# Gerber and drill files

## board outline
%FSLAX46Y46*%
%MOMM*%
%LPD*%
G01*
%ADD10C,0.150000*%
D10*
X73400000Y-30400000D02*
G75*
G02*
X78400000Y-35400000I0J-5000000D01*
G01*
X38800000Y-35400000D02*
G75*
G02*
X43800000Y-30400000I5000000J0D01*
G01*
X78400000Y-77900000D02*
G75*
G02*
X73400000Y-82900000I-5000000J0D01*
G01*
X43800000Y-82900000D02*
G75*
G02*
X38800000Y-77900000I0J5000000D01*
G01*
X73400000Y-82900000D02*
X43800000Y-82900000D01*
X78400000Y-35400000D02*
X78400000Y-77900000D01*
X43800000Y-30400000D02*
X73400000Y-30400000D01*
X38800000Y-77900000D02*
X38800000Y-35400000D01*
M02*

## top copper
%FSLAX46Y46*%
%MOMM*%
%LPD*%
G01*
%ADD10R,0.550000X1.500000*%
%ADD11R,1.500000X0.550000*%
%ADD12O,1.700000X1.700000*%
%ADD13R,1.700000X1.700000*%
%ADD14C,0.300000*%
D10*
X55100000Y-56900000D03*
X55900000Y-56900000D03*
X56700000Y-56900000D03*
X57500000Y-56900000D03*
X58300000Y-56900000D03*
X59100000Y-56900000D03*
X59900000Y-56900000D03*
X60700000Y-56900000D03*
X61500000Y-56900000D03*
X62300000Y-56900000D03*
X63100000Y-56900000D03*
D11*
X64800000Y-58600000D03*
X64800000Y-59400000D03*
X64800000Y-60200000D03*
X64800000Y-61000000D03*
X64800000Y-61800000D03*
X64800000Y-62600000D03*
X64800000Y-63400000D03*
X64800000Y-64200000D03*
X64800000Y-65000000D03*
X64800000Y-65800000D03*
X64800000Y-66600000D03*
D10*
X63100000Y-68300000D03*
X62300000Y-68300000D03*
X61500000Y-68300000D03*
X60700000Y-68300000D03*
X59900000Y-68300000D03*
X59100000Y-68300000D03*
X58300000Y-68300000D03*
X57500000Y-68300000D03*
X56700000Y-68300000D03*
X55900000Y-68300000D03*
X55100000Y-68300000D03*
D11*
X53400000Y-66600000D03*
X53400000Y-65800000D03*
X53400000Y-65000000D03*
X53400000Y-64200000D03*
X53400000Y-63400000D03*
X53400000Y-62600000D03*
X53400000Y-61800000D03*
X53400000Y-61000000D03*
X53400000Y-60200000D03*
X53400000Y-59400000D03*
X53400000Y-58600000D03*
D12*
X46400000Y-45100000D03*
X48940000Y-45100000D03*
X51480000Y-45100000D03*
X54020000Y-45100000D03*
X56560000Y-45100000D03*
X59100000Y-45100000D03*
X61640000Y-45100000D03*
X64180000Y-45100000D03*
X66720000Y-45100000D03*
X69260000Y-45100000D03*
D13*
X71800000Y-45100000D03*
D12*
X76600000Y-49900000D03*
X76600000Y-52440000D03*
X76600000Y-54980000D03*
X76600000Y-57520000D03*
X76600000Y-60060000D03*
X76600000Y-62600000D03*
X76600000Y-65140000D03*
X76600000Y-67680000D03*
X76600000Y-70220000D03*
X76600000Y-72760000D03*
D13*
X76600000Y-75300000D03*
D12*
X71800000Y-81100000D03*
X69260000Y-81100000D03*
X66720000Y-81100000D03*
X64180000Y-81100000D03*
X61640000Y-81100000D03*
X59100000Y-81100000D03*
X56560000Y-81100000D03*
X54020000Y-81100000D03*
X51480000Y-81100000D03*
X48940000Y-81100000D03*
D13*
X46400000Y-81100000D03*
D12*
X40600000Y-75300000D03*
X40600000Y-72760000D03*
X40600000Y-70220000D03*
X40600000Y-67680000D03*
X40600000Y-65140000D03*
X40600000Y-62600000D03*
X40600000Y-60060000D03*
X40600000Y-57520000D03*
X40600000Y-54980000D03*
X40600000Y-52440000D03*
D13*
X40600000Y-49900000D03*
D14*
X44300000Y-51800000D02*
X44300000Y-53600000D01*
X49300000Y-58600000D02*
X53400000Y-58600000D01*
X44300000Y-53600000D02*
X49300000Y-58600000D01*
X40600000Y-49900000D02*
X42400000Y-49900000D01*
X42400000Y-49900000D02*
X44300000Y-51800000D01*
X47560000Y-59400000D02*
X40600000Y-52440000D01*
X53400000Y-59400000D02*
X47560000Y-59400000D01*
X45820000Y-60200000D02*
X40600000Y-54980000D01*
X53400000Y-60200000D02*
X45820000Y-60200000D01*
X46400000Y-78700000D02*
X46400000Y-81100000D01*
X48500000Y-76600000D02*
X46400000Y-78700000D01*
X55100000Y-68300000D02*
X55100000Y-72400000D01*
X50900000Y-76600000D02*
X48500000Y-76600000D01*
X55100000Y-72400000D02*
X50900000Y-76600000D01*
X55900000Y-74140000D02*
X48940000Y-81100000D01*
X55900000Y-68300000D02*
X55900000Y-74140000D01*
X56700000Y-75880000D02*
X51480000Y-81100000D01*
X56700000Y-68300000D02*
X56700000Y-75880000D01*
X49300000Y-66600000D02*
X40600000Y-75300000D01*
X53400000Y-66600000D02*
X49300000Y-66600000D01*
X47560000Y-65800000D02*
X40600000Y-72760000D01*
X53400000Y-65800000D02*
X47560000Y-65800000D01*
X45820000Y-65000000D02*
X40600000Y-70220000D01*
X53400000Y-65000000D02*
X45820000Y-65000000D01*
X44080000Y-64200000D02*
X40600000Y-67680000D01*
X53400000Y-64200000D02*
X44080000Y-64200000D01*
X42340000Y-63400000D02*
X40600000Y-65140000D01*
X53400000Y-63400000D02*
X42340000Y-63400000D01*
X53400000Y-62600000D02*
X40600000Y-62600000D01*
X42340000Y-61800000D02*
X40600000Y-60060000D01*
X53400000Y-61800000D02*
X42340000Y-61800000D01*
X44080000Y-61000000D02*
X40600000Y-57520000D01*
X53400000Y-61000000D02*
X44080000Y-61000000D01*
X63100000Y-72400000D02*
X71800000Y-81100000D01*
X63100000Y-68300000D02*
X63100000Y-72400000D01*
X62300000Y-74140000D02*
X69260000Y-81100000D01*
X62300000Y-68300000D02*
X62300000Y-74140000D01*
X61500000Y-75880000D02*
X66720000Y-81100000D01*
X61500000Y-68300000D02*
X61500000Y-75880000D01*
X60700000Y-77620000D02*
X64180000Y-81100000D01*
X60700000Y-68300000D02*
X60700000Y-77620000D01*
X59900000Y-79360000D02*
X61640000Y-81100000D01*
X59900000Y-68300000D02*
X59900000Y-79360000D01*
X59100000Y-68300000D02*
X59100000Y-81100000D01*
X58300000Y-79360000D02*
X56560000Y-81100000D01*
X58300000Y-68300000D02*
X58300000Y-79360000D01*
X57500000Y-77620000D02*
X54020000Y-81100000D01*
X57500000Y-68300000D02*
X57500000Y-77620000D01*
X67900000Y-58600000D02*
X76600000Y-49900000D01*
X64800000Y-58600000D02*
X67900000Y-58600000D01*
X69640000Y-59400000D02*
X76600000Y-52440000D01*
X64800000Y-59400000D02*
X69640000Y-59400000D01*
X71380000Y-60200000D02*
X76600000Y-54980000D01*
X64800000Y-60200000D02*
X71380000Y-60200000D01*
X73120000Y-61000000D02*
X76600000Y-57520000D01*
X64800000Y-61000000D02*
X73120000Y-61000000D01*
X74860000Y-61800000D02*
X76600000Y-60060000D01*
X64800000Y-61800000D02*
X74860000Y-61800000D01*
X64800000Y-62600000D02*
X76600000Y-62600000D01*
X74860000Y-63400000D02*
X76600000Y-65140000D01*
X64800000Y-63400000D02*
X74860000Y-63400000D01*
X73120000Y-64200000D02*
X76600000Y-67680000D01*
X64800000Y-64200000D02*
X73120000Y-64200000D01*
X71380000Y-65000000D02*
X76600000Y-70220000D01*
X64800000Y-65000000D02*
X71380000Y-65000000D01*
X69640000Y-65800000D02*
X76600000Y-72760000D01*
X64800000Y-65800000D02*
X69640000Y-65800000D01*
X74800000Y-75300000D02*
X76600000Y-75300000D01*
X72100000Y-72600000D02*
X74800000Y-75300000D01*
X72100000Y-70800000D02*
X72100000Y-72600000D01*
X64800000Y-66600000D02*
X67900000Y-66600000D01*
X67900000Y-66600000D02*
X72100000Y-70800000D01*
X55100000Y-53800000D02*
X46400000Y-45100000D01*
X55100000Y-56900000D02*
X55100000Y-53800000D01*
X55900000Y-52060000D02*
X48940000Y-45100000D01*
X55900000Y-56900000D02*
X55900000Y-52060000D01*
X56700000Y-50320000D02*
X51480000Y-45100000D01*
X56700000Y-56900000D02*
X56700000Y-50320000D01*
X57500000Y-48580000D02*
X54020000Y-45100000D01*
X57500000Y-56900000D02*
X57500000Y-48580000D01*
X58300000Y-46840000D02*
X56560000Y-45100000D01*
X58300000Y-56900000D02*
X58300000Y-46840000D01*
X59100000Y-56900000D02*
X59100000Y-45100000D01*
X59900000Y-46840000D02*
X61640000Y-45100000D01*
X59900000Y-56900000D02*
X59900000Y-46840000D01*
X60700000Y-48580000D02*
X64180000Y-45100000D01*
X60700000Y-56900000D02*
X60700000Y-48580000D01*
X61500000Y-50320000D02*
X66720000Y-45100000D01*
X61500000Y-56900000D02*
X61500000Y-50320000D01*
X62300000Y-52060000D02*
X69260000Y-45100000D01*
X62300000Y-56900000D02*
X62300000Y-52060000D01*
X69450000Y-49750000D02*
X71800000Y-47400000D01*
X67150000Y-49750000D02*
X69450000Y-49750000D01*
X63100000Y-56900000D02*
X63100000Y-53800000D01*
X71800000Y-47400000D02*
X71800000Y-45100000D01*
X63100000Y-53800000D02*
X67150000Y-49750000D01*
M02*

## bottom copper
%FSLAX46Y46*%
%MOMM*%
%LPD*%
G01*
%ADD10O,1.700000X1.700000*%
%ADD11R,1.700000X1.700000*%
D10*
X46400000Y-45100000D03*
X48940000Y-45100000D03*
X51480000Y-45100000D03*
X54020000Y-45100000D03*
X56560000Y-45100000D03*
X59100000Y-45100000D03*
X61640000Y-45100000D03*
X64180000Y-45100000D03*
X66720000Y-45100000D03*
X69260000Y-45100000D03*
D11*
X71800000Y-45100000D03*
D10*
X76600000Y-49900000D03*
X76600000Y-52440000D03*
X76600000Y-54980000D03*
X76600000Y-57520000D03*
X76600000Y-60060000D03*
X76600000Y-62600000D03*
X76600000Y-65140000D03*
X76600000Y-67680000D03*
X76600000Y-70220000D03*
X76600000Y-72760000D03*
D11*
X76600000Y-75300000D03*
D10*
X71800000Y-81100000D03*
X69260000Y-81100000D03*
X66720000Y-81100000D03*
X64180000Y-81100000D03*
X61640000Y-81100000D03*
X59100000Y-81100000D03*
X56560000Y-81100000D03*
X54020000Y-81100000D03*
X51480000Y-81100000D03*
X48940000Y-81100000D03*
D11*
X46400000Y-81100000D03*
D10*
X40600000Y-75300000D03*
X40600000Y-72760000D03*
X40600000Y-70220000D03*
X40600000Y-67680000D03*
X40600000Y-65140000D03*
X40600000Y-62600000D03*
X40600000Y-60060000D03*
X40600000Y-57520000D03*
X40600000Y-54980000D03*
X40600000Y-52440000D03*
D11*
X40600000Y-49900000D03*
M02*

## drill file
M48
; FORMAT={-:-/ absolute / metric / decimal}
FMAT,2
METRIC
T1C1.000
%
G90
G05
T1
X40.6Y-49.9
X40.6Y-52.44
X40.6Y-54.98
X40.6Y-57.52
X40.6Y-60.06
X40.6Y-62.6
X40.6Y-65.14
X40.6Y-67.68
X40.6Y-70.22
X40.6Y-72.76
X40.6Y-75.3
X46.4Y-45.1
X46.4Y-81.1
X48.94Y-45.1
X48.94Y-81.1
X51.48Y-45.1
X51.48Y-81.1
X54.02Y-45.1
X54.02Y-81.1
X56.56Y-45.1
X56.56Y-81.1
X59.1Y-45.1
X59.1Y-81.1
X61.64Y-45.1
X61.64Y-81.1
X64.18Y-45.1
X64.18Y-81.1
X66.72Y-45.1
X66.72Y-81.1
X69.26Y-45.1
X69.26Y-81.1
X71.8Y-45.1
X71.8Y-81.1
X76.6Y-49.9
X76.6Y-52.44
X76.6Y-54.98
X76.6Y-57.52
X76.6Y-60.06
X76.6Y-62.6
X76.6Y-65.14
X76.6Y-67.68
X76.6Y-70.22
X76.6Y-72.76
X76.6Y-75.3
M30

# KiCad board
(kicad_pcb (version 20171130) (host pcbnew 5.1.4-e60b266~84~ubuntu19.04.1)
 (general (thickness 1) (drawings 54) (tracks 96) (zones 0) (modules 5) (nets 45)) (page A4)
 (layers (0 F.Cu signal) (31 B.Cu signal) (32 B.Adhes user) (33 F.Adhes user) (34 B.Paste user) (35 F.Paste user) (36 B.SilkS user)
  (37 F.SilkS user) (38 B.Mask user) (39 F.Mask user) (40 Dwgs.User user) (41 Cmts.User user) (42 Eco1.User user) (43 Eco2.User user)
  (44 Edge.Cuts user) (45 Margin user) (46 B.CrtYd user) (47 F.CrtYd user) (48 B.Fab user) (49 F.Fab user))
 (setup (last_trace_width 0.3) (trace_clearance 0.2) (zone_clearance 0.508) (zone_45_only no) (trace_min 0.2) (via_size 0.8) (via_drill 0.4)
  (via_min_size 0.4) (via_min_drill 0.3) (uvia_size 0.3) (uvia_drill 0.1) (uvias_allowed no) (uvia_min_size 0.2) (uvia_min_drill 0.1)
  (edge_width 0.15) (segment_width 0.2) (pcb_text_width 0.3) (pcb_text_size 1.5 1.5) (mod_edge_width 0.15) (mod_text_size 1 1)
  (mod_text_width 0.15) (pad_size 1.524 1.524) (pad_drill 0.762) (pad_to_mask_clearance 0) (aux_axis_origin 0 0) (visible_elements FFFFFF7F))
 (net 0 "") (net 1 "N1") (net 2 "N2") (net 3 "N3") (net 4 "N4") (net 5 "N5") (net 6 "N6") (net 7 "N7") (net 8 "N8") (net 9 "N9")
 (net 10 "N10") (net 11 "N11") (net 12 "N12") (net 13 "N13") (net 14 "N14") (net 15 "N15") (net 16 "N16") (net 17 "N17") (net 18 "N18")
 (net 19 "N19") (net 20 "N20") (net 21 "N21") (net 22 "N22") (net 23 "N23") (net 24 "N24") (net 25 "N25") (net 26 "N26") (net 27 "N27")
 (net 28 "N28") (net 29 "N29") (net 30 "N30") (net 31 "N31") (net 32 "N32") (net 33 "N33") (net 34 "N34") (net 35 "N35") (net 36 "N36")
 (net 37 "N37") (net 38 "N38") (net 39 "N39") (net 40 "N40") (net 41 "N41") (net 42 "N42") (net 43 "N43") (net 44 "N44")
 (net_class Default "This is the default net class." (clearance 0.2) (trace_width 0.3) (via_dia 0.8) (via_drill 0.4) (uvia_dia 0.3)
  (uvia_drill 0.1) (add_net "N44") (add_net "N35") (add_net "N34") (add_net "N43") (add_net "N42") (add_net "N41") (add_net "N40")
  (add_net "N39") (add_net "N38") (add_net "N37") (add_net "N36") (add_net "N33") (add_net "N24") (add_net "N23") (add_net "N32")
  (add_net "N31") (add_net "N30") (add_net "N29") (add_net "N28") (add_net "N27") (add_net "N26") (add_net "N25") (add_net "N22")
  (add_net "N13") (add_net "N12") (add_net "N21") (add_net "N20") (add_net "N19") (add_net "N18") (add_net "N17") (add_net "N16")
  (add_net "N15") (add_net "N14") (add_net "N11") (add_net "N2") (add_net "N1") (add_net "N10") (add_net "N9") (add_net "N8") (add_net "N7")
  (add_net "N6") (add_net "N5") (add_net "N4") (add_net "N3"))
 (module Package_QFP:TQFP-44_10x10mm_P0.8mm (layer F.Cu) (at 59.1 62.6)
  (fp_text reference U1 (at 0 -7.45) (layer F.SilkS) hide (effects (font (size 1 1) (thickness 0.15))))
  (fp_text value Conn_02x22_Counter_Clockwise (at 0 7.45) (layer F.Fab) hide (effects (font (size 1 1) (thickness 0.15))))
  (pad 44 smd rect (at -4 -5.7 90) (size 1.5 0.55) (layers F.Cu F.Paste F.Mask) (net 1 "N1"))
  (pad 43 smd rect (at -3.2 -5.7 90) (size 1.5 0.55) (layers F.Cu F.Paste F.Mask) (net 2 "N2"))
  (pad 42 smd rect (at -2.4 -5.7 90) (size 1.5 0.55) (layers F.Cu F.Paste F.Mask) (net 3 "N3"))
  (pad 41 smd rect (at -1.6 -5.7 90) (size 1.5 0.55) (layers F.Cu F.Paste F.Mask) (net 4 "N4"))
  (pad 40 smd rect (at -0.8 -5.7 90) (size 1.5 0.55) (layers F.Cu F.Paste F.Mask) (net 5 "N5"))
  (pad 39 smd rect (at 0 -5.7 90) (size 1.5 0.55) (layers F.Cu F.Paste F.Mask) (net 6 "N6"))
  (pad 38 smd rect (at 0.8 -5.7 90) (size 1.5 0.55) (layers F.Cu F.Paste F.Mask) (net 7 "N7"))
  (pad 37 smd rect (at 1.6 -5.7 90) (size 1.5 0.55) (layers F.Cu F.Paste F.Mask) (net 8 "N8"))
  (pad 36 smd rect (at 2.4 -5.7 90) (size 1.5 0.55) (layers F.Cu F.Paste F.Mask) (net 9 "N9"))
  (pad 35 smd rect (at 3.2 -5.7 90) (size 1.5 0.55) (layers F.Cu F.Paste F.Mask) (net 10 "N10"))
  (pad 34 smd rect (at 4 -5.7 90) (size 1.5 0.55) (layers F.Cu F.Paste F.Mask) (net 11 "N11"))
  (pad 33 smd rect (at 5.7 -4) (size 1.5 0.55) (layers F.Cu F.Paste F.Mask) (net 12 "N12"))
  (pad 32 smd rect (at 5.7 -3.2) (size 1.5 0.55) (layers F.Cu F.Paste F.Mask) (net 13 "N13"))
  (pad 31 smd rect (at 5.7 -2.4) (size 1.5 0.55) (layers F.Cu F.Paste F.Mask) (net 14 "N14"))
  (pad 30 smd rect (at 5.7 -1.6) (size 1.5 0.55) (layers F.Cu F.Paste F.Mask) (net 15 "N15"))
  (pad 29 smd rect (at 5.7 -0.8) (size 1.5 0.55) (layers F.Cu F.Paste F.Mask) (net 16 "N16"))
  (pad 28 smd rect (at 5.7 0) (size 1.5 0.55) (layers F.Cu F.Paste F.Mask) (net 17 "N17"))
  (pad 27 smd rect (at 5.7 0.8) (size 1.5 0.55) (layers F.Cu F.Paste F.Mask) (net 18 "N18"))
  (pad 26 smd rect (at 5.7 1.6) (size 1.5 0.55) (layers F.Cu F.Paste F.Mask) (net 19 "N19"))
  (pad 25 smd rect (at 5.7 2.4) (size 1.5 0.55) (layers F.Cu F.Paste F.Mask) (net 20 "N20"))
  (pad 24 smd rect (at 5.7 3.2) (size 1.5 0.55) (layers F.Cu F.Paste F.Mask) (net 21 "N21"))
  (pad 23 smd rect (at 5.7 4) (size 1.5 0.55) (layers F.Cu F.Paste F.Mask) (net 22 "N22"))
  (pad 22 smd rect (at 4 5.7 90) (size 1.5 0.55) (layers F.Cu F.Paste F.Mask) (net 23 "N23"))
  (pad 21 smd rect (at 3.2 5.7 90) (size 1.5 0.55) (layers F.Cu F.Paste F.Mask) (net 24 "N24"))
  (pad 20 smd rect (at 2.4 5.7 90) (size 1.5 0.55) (layers F.Cu F.Paste F.Mask) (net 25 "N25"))
  (pad 19 smd rect (at 1.6 5.7 90) (size 1.5 0.55) (layers F.Cu F.Paste F.Mask) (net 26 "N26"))
  (pad 18 smd rect (at 0.8 5.7 90) (size 1.5 0.55) (layers F.Cu F.Paste F.Mask) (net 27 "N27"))
  (pad 17 smd rect (at 0 5.7 90) (size 1.5 0.55) (layers F.Cu F.Paste F.Mask) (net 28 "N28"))
  (pad 16 smd rect (at -0.8 5.7 90) (size 1.5 0.55) (layers F.Cu F.Paste F.Mask) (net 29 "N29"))
  (pad 15 smd rect (at -1.6 5.7 90) (size 1.5 0.55) (layers F.Cu F.Paste F.Mask) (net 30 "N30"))
  (pad 14 smd rect (at -2.4 5.7 90) (size 1.5 0.55) (layers F.Cu F.Paste F.Mask) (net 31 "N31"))
  (pad 13 smd rect (at -3.2 5.7 90) (size 1.5 0.55) (layers F.Cu F.Paste F.Mask) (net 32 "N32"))
  (pad 12 smd rect (at -4 5.7 90) (size 1.5 0.55) (layers F.Cu F.Paste F.Mask) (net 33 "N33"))
  (pad 11 smd rect (at -5.7 4) (size 1.5 0.55) (layers F.Cu F.Paste F.Mask) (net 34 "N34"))
  (pad 10 smd rect (at -5.7 3.2) (size 1.5 0.55) (layers F.Cu F.Paste F.Mask) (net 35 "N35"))
  (pad 9 smd rect (at -5.7 2.4) (size 1.5 0.55) (layers F.Cu F.Paste F.Mask) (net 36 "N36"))
  (pad 8 smd rect (at -5.7 1.6) (size 1.5 0.55) (layers F.Cu F.Paste F.Mask) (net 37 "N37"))
  (pad 7 smd rect (at -5.7 0.8) (size 1.5 0.55) (layers F.Cu F.Paste F.Mask) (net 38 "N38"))
  (pad 6 smd rect (at -5.7 0) (size 1.5 0.55) (layers F.Cu F.Paste F.Mask) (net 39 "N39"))
  (pad 5 smd rect (at -5.7 -0.8) (size 1.5 0.55) (layers F.Cu F.Paste F.Mask) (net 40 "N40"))
  (pad 4 smd rect (at -5.7 -1.6) (size 1.5 0.55) (layers F.Cu F.Paste F.Mask) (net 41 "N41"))
  (pad 3 smd rect (at -5.7 -2.4) (size 1.5 0.55) (layers F.Cu F.Paste F.Mask) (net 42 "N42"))
  (pad 2 smd rect (at -5.7 -3.2) (size 1.5 0.55) (layers F.Cu F.Paste F.Mask) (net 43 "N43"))
  (pad 1 smd rect (at -5.7 -4) (size 1.5 0.55) (layers F.Cu F.Paste F.Mask) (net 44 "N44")))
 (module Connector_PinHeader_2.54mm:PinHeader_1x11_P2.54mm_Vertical (layer F.Cu) (at 71.8 45.1 270)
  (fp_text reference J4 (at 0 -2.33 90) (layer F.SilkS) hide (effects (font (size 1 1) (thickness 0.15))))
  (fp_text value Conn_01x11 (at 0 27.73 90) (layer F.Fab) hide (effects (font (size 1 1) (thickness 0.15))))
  (pad 11 thru_hole oval (at 0 25.4 270) (size 1.7 1.7) (drill 1) (layers *.Cu *.Mask) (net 1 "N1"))
  (pad 10 thru_hole oval (at 0 22.86 270) (size 1.7 1.7) (drill 1) (layers *.Cu *.Mask) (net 2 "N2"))
  (pad 9 thru_hole oval (at 0 20.32 270) (size 1.7 1.7) (drill 1) (layers *.Cu *.Mask) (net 3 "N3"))
  (pad 8 thru_hole oval (at 0 17.78 270) (size 1.7 1.7) (drill 1) (layers *.Cu *.Mask) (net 4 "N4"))
  (pad 7 thru_hole oval (at 0 15.24 270) (size 1.7 1.7) (drill 1) (layers *.Cu *.Mask) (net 5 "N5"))
  (pad 6 thru_hole oval (at 0 12.7 270) (size 1.7 1.7) (drill 1) (layers *.Cu *.Mask) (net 6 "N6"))
  (pad 5 thru_hole oval (at 0 10.16 270) (size 1.7 1.7) (drill 1) (layers *.Cu *.Mask) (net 7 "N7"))
  (pad 4 thru_hole oval (at 0 7.62 270) (size 1.7 1.7) (drill 1) (layers *.Cu *.Mask) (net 8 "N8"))
  (pad 3 thru_hole oval (at 0 5.08 270) (size 1.7 1.7) (drill 1) (layers *.Cu *.Mask) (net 9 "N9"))
  (pad 2 thru_hole oval (at 0 2.54 270) (size 1.7 1.7) (drill 1) (layers *.Cu *.Mask) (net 10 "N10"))
  (pad 1 thru_hole rect (at 0 0 270) (size 1.7 1.7) (drill 1) (layers *.Cu *.Mask) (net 11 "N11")))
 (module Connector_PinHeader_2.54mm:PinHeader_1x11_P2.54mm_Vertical (layer F.Cu) (at 76.6 75.3 180)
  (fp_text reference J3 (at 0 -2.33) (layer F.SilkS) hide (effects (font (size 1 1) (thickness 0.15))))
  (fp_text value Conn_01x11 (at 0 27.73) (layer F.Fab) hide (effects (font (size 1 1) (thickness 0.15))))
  (pad 11 thru_hole oval (at 0 25.4 180) (size 1.7 1.7) (drill 1) (layers *.Cu *.Mask) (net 12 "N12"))
  (pad 10 thru_hole oval (at 0 22.86 180) (size 1.7 1.7) (drill 1) (layers *.Cu *.Mask) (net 13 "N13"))
  (pad 9 thru_hole oval (at 0 20.32 180) (size 1.7 1.7) (drill 1) (layers *.Cu *.Mask) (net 14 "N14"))
  (pad 8 thru_hole oval (at 0 17.78 180) (size 1.7 1.7) (drill 1) (layers *.Cu *.Mask) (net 15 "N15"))
  (pad 7 thru_hole oval (at 0 15.24 180) (size 1.7 1.7) (drill 1) (layers *.Cu *.Mask) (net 16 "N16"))
  (pad 6 thru_hole oval (at 0 12.7 180) (size 1.7 1.7) (drill 1) (layers *.Cu *.Mask) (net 17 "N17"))
  (pad 5 thru_hole oval (at 0 10.16 180) (size 1.7 1.7) (drill 1) (layers *.Cu *.Mask) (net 18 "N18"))
  (pad 4 thru_hole oval (at 0 7.62 180) (size 1.7 1.7) (drill 1) (layers *.Cu *.Mask) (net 19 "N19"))
  (pad 3 thru_hole oval (at 0 5.08 180) (size 1.7 1.7) (drill 1) (layers *.Cu *.Mask) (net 20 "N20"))
  (pad 2 thru_hole oval (at 0 2.54 180) (size 1.7 1.7) (drill 1) (layers *.Cu *.Mask) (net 21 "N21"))
  (pad 1 thru_hole rect (at 0 0 180) (size 1.7 1.7) (drill 1) (layers *.Cu *.Mask) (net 22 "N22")))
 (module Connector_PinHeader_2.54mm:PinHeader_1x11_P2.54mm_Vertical (layer F.Cu) (at 46.4 81.1 90)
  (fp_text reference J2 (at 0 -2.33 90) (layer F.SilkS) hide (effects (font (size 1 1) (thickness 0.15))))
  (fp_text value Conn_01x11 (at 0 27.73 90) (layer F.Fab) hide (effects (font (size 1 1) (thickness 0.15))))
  (pad 11 thru_hole oval (at 0 25.4 90) (size 1.7 1.7) (drill 1) (layers *.Cu *.Mask) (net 23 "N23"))
  (pad 10 thru_hole oval (at 0 22.86 90) (size 1.7 1.7) (drill 1) (layers *.Cu *.Mask) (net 24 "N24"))
  (pad 9 thru_hole oval (at 0 20.32 90) (size 1.7 1.7) (drill 1) (layers *.Cu *.Mask) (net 25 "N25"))
  (pad 8 thru_hole oval (at 0 17.78 90) (size 1.7 1.7) (drill 1) (layers *.Cu *.Mask) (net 26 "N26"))
  (pad 7 thru_hole oval (at 0 15.24 90) (size 1.7 1.7) (drill 1) (layers *.Cu *.Mask) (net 27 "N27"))
  (pad 6 thru_hole oval (at 0 12.7 90) (size 1.7 1.7) (drill 1) (layers *.Cu *.Mask) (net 28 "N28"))
  (pad 5 thru_hole oval (at 0 10.16 90) (size 1.7 1.7) (drill 1) (layers *.Cu *.Mask) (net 29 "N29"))
  (pad 4 thru_hole oval (at 0 7.62 90) (size 1.7 1.7) (drill 1) (layers *.Cu *.Mask) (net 30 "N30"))
  (pad 3 thru_hole oval (at 0 5.08 90) (size 1.7 1.7) (drill 1) (layers *.Cu *.Mask) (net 31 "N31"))
  (pad 2 thru_hole oval (at 0 2.54 90) (size 1.7 1.7) (drill 1) (layers *.Cu *.Mask) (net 32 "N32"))
  (pad 1 thru_hole rect (at 0 0 90) (size 1.7 1.7) (drill 1) (layers *.Cu *.Mask) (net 33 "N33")))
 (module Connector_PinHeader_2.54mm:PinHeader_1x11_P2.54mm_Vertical (layer F.Cu) (at 40.6 49.9)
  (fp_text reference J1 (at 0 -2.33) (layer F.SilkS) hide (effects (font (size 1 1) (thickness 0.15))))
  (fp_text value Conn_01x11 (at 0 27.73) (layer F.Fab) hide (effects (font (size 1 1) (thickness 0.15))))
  (pad 11 thru_hole oval (at 0 25.4) (size 1.7 1.7) (drill 1) (layers *.Cu *.Mask) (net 34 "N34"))
  (pad 10 thru_hole oval (at 0 22.86) (size 1.7 1.7) (drill 1) (layers *.Cu *.Mask) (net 35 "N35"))
  (pad 9 thru_hole oval (at 0 20.32) (size 1.7 1.7) (drill 1) (layers *.Cu *.Mask) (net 36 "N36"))
  (pad 8 thru_hole oval (at 0 17.78) (size 1.7 1.7) (drill 1) (layers *.Cu *.Mask) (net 37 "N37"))
  (pad 7 thru_hole oval (at 0 15.24) (size 1.7 1.7) (drill 1) (layers *.Cu *.Mask) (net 38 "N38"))
  (pad 6 thru_hole oval (at 0 12.7) (size 1.7 1.7) (drill 1) (layers *.Cu *.Mask) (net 39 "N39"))
  (pad 5 thru_hole oval (at 0 10.16) (size 1.7 1.7) (drill 1) (layers *.Cu *.Mask) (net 40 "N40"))
  (pad 4 thru_hole oval (at 0 7.62) (size 1.7 1.7) (drill 1) (layers *.Cu *.Mask) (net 41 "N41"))
  (pad 3 thru_hole oval (at 0 5.08) (size 1.7 1.7) (drill 1) (layers *.Cu *.Mask) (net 42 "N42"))
  (pad 2 thru_hole oval (at 0 2.54) (size 1.7 1.7) (drill 1) (layers *.Cu *.Mask) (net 43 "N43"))
  (pad 1 thru_hole rect (at 0 0) (size 1.7 1.7) (drill 1) (layers *.Cu *.Mask) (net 44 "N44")))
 (gr_arc (start 73.4 35.4) (end 78.4 35.4) (angle -90) (layer Edge.Cuts) (width 0.15))
 (gr_arc (start 43.8 35.4) (end 43.8 30.4) (angle -90) (layer Edge.Cuts) (width 0.15))
 (gr_arc (start 73.4 77.9) (end 73.4 82.9) (angle -90) (layer Edge.Cuts) (width 0.15))
 (gr_arc (start 43.8 77.9) (end 38.8 77.9) (angle -90) (layer Edge.Cuts) (width 0.15))
 (gr_line (start 73.4 82.9) (end 43.8 82.9) (layer Edge.Cuts) (width 0.15))
 (gr_line (start 78.4 35.4) (end 78.4 77.9) (layer Edge.Cuts) (width 0.15))
 (gr_line (start 43.8 30.4) (end 73.4 30.4) (layer Edge.Cuts) (width 0.15))
 (gr_line (start 38.8 77.9) (end 38.8 35.4) (layer Edge.Cuts) (width 0.15))
 (segment (start 44.3 51.8) (end 44.3 53.6) (width 0.3) (layer F.Cu) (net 44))
 (segment (start 49.3 58.6) (end 53.4 58.6) (width 0.3) (layer F.Cu) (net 44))
 (segment (start 44.3 53.6) (end 49.3 58.6) (width 0.3) (layer F.Cu) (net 44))
 (segment (start 40.6 49.9) (end 42.4 49.9) (width 0.3) (layer F.Cu) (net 44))
 (segment (start 42.4 49.9) (end 44.3 51.8) (width 0.3) (layer F.Cu) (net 44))
 (segment (start 47.56 59.4) (end 40.6 52.44) (width 0.3) (layer F.Cu) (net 43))
 (segment (start 53.4 59.4) (end 47.56 59.4) (width 0.3) (layer F.Cu) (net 43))
 (segment (start 45.82 60.2) (end 40.6 54.98) (width 0.3) (layer F.Cu) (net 42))
 (segment (start 53.4 60.2) (end 45.82 60.2) (width 0.3) (layer F.Cu) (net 42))
 (segment (start 46.4 78.7) (end 46.4 81.1) (width 0.3) (layer F.Cu) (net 33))
 (segment (start 48.5 76.6) (end 46.4 78.7) (width 0.3) (layer F.Cu) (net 33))
 (segment (start 55.1 68.3) (end 55.1 72.4) (width 0.3) (layer F.Cu) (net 33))
 (segment (start 50.9 76.6) (end 48.5 76.6) (width 0.3) (layer F.Cu) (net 33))
 (segment (start 55.1 72.4) (end 50.9 76.6) (width 0.3) (layer F.Cu) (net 33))
 (segment (start 55.9 74.14) (end 48.94 81.1) (width 0.3) (layer F.Cu) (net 32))
 (segment (start 55.9 68.3) (end 55.9 74.14) (width 0.3) (layer F.Cu) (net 32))
 (segment (start 56.7 75.88) (end 51.48 81.1) (width 0.3) (layer F.Cu) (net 31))
 (segment (start 56.7 68.3) (end 56.7 75.88) (width 0.3) (layer F.Cu) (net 31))
 (segment (start 49.3 66.6) (end 40.6 75.3) (width 0.3) (layer F.Cu) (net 34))
 (segment (start 53.4 66.6) (end 49.3 66.6) (width 0.3) (layer F.Cu) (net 34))
 (segment (start 47.56 65.8) (end 40.6 72.76) (width 0.3) (layer F.Cu) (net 35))
 (segment (start 53.4 65.8) (end 47.56 65.8) (width 0.3) (layer F.Cu) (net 35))
 (segment (start 45.82 65) (end 40.6 70.22) (width 0.3) (layer F.Cu) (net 36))
 (segment (start 53.4 65) (end 45.82 65) (width 0.3) (layer F.Cu) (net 36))
 (segment (start 44.08 64.2) (end 40.6 67.68) (width 0.3) (layer F.Cu) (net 37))
 (segment (start 53.4 64.2) (end 44.08 64.2) (width 0.3) (layer F.Cu) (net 37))
 (segment (start 42.34 63.4) (end 40.6 65.14) (width 0.3) (layer F.Cu) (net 38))
 (segment (start 53.4 63.4) (end 42.34 63.4) (width 0.3) (layer F.Cu) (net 38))
 (segment (start 53.4 62.6) (end 40.6 62.6) (width 0.3) (layer F.Cu) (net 39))
 (segment (start 42.34 61.8) (end 40.6 60.06) (width 0.3) (layer F.Cu) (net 40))
 (segment (start 53.4 61.8) (end 42.34 61.8) (width 0.3) (layer F.Cu) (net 40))
 (segment (start 44.08 61) (end 40.6 57.52) (width 0.3) (layer F.Cu) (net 41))
 (segment (start 53.4 61) (end 44.08 61) (width 0.3) (layer F.Cu) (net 41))
 (segment (start 63.1 72.4) (end 71.8 81.1) (width 0.3) (layer F.Cu) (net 23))
 (segment (start 63.1 68.3) (end 63.1 72.4) (width 0.3) (layer F.Cu) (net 23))
 (segment (start 62.3 74.14) (end 69.26 81.1) (width 0.3) (layer F.Cu) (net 24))
 (segment (start 62.3 68.3) (end 62.3 74.14) (width 0.3) (layer F.Cu) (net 24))
 (segment (start 61.5 75.88) (end 66.72 81.1) (width 0.3) (layer F.Cu) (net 25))
 (segment (start 61.5 68.3) (end 61.5 75.88) (width 0.3) (layer F.Cu) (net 25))
 (segment (start 60.7 77.62) (end 64.18 81.1) (width 0.3) (layer F.Cu) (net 26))
 (segment (start 60.7 68.3) (end 60.7 77.62) (width 0.3) (layer F.Cu) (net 26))
 (segment (start 59.9 79.36) (end 61.64 81.1) (width 0.3) (layer F.Cu) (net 27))
 (segment (start 59.9 68.3) (end 59.9 79.36) (width 0.3) (layer F.Cu) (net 27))
 (segment (start 59.1 68.3) (end 59.1 81.1) (width 0.3) (layer F.Cu) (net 28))
 (segment (start 58.3 79.36) (end 56.56 81.1) (width 0.3) (layer F.Cu) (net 29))
 (segment (start 58.3 68.3) (end 58.3 79.36) (width 0.3) (layer F.Cu) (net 29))
 (segment (start 57.5 77.62) (end 54.02 81.1) (width 0.3) (layer F.Cu) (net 30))
 (segment (start 57.5 68.3) (end 57.5 77.62) (width 0.3) (layer F.Cu) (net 30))
 (segment (start 67.9 58.6) (end 76.6 49.9) (width 0.3) (layer F.Cu) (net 12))
 (segment (start 64.8 58.6) (end 67.9 58.6) (width 0.3) (layer F.Cu) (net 12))
 (segment (start 69.64 59.4) (end 76.6 52.44) (width 0.3) (layer F.Cu) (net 13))
 (segment (start 64.8 59.4) (end 69.64 59.4) (width 0.3) (layer F.Cu) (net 13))
 (segment (start 71.38 60.2) (end 76.6 54.98) (width 0.3) (layer F.Cu) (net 14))
 (segment (start 64.8 60.2) (end 71.38 60.2) (width 0.3) (layer F.Cu) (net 14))
 (segment (start 73.12 61) (end 76.6 57.52) (width 0.3) (layer F.Cu) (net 15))
 (segment (start 64.8 61) (end 73.12 61) (width 0.3) (layer F.Cu) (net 15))
 (segment (start 74.86 61.8) (end 76.6 60.06) (width 0.3) (layer F.Cu) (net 16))
 (segment (start 64.8 61.8) (end 74.86 61.8) (width 0.3) (layer F.Cu) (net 16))
 (segment (start 64.8 62.6) (end 76.6 62.6) (width 0.3) (layer F.Cu) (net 17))
 (segment (start 74.86 63.4) (end 76.6 65.14) (width 0.3) (layer F.Cu) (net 18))
 (segment (start 64.8 63.4) (end 74.86 63.4) (width 0.3) (layer F.Cu) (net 18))
 (segment (start 73.12 64.2) (end 76.6 67.68) (width 0.3) (layer F.Cu) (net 19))
 (segment (start 64.8 64.2) (end 73.12 64.2) (width 0.3) (layer F.Cu) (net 19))
 (segment (start 71.38 65) (end 76.6 70.22) (width 0.3) (layer F.Cu) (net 20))
 (segment (start 64.8 65) (end 71.38 65) (width 0.3) (layer F.Cu) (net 20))
 (segment (start 69.64 65.8) (end 76.6 72.76) (width 0.3) (layer F.Cu) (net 21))
 (segment (start 64.8 65.8) (end 69.64 65.8) (width 0.3) (layer F.Cu) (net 21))
 (segment (start 74.8 75.3) (end 76.6 75.3) (width 0.3) (layer F.Cu) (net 22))
 (segment (start 72.1 72.6) (end 74.8 75.3) (width 0.3) (layer F.Cu) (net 22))
 (segment (start 72.1 70.8) (end 72.1 72.6) (width 0.3) (layer F.Cu) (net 22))
 (segment (start 64.8 66.6) (end 67.9 66.6) (width 0.3) (layer F.Cu) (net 22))
 (segment (start 67.9 66.6) (end 72.1 70.8) (width 0.3) (layer F.Cu) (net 22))
 (segment (start 55.1 53.8) (end 46.4 45.1) (width 0.3) (layer F.Cu) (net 1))
 (segment (start 55.1 56.9) (end 55.1 53.8) (width 0.3) (layer F.Cu) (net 1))
 (segment (start 55.9 52.06) (end 48.94 45.1) (width 0.3) (layer F.Cu) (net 2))
 (segment (start 55.9 56.9) (end 55.9 52.06) (width 0.3) (layer F.Cu) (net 2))
 (segment (start 56.7 50.32) (end 51.48 45.1) (width 0.3) (layer F.Cu) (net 3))
 (segment (start 56.7 56.9) (end 56.7 50.32) (width 0.3) (layer F.Cu) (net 3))
 (segment (start 57.5 48.58) (end 54.02 45.1) (width 0.3) (layer F.Cu) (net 4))
 (segment (start 57.5 56.9) (end 57.5 48.58) (width 0.3) (layer F.Cu) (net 4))
 (segment (start 58.3 46.84) (end 56.56 45.1) (width 0.3) (layer F.Cu) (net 5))
 (segment (start 58.3 56.9) (end 58.3 46.84) (width 0.3) (layer F.Cu) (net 5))
 (segment (start 59.1 56.9) (end 59.1 45.1) (width 0.3) (layer F.Cu) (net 6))
 (segment (start 59.9 46.84) (end 61.64 45.1) (width 0.3) (layer F.Cu) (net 7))
 (segment (start 59.9 56.9) (end 59.9 46.84) (width 0.3) (layer F.Cu) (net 7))
 (segment (start 60.7 48.58) (end 64.18 45.1) (width 0.3) (layer F.Cu) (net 8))
 (segment (start 60.7 56.9) (end 60.7 48.58) (width 0.3) (layer F.Cu) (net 8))
 (segment (start 61.5 50.32) (end 66.72 45.1) (width 0.3) (layer F.Cu) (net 9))
 (segment (start 61.5 56.9) (end 61.5 50.32) (width 0.3) (layer F.Cu) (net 9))
 (segment (start 62.3 52.06) (end 69.26 45.1) (width 0.3) (layer F.Cu) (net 10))
 (segment (start 62.3 56.9) (end 62.3 52.06) (width 0.3) (layer F.Cu) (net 10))
 (segment (start 69.45 49.75) (end 71.8 47.4) (width 0.3) (layer F.Cu) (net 11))
 (segment (start 67.15 49.75) (end 69.45 49.75) (width 0.3) (layer F.Cu) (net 11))
 (segment (start 63.1 56.9) (end 63.1 53.8) (width 0.3) (layer F.Cu) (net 11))
 (segment (start 71.8 47.4) (end 71.8 45.1) (width 0.3) (layer F.Cu) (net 11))
 (segment (start 63.1 53.8) (end 67.15 49.75) (width 0.3) (layer F.Cu) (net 11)))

